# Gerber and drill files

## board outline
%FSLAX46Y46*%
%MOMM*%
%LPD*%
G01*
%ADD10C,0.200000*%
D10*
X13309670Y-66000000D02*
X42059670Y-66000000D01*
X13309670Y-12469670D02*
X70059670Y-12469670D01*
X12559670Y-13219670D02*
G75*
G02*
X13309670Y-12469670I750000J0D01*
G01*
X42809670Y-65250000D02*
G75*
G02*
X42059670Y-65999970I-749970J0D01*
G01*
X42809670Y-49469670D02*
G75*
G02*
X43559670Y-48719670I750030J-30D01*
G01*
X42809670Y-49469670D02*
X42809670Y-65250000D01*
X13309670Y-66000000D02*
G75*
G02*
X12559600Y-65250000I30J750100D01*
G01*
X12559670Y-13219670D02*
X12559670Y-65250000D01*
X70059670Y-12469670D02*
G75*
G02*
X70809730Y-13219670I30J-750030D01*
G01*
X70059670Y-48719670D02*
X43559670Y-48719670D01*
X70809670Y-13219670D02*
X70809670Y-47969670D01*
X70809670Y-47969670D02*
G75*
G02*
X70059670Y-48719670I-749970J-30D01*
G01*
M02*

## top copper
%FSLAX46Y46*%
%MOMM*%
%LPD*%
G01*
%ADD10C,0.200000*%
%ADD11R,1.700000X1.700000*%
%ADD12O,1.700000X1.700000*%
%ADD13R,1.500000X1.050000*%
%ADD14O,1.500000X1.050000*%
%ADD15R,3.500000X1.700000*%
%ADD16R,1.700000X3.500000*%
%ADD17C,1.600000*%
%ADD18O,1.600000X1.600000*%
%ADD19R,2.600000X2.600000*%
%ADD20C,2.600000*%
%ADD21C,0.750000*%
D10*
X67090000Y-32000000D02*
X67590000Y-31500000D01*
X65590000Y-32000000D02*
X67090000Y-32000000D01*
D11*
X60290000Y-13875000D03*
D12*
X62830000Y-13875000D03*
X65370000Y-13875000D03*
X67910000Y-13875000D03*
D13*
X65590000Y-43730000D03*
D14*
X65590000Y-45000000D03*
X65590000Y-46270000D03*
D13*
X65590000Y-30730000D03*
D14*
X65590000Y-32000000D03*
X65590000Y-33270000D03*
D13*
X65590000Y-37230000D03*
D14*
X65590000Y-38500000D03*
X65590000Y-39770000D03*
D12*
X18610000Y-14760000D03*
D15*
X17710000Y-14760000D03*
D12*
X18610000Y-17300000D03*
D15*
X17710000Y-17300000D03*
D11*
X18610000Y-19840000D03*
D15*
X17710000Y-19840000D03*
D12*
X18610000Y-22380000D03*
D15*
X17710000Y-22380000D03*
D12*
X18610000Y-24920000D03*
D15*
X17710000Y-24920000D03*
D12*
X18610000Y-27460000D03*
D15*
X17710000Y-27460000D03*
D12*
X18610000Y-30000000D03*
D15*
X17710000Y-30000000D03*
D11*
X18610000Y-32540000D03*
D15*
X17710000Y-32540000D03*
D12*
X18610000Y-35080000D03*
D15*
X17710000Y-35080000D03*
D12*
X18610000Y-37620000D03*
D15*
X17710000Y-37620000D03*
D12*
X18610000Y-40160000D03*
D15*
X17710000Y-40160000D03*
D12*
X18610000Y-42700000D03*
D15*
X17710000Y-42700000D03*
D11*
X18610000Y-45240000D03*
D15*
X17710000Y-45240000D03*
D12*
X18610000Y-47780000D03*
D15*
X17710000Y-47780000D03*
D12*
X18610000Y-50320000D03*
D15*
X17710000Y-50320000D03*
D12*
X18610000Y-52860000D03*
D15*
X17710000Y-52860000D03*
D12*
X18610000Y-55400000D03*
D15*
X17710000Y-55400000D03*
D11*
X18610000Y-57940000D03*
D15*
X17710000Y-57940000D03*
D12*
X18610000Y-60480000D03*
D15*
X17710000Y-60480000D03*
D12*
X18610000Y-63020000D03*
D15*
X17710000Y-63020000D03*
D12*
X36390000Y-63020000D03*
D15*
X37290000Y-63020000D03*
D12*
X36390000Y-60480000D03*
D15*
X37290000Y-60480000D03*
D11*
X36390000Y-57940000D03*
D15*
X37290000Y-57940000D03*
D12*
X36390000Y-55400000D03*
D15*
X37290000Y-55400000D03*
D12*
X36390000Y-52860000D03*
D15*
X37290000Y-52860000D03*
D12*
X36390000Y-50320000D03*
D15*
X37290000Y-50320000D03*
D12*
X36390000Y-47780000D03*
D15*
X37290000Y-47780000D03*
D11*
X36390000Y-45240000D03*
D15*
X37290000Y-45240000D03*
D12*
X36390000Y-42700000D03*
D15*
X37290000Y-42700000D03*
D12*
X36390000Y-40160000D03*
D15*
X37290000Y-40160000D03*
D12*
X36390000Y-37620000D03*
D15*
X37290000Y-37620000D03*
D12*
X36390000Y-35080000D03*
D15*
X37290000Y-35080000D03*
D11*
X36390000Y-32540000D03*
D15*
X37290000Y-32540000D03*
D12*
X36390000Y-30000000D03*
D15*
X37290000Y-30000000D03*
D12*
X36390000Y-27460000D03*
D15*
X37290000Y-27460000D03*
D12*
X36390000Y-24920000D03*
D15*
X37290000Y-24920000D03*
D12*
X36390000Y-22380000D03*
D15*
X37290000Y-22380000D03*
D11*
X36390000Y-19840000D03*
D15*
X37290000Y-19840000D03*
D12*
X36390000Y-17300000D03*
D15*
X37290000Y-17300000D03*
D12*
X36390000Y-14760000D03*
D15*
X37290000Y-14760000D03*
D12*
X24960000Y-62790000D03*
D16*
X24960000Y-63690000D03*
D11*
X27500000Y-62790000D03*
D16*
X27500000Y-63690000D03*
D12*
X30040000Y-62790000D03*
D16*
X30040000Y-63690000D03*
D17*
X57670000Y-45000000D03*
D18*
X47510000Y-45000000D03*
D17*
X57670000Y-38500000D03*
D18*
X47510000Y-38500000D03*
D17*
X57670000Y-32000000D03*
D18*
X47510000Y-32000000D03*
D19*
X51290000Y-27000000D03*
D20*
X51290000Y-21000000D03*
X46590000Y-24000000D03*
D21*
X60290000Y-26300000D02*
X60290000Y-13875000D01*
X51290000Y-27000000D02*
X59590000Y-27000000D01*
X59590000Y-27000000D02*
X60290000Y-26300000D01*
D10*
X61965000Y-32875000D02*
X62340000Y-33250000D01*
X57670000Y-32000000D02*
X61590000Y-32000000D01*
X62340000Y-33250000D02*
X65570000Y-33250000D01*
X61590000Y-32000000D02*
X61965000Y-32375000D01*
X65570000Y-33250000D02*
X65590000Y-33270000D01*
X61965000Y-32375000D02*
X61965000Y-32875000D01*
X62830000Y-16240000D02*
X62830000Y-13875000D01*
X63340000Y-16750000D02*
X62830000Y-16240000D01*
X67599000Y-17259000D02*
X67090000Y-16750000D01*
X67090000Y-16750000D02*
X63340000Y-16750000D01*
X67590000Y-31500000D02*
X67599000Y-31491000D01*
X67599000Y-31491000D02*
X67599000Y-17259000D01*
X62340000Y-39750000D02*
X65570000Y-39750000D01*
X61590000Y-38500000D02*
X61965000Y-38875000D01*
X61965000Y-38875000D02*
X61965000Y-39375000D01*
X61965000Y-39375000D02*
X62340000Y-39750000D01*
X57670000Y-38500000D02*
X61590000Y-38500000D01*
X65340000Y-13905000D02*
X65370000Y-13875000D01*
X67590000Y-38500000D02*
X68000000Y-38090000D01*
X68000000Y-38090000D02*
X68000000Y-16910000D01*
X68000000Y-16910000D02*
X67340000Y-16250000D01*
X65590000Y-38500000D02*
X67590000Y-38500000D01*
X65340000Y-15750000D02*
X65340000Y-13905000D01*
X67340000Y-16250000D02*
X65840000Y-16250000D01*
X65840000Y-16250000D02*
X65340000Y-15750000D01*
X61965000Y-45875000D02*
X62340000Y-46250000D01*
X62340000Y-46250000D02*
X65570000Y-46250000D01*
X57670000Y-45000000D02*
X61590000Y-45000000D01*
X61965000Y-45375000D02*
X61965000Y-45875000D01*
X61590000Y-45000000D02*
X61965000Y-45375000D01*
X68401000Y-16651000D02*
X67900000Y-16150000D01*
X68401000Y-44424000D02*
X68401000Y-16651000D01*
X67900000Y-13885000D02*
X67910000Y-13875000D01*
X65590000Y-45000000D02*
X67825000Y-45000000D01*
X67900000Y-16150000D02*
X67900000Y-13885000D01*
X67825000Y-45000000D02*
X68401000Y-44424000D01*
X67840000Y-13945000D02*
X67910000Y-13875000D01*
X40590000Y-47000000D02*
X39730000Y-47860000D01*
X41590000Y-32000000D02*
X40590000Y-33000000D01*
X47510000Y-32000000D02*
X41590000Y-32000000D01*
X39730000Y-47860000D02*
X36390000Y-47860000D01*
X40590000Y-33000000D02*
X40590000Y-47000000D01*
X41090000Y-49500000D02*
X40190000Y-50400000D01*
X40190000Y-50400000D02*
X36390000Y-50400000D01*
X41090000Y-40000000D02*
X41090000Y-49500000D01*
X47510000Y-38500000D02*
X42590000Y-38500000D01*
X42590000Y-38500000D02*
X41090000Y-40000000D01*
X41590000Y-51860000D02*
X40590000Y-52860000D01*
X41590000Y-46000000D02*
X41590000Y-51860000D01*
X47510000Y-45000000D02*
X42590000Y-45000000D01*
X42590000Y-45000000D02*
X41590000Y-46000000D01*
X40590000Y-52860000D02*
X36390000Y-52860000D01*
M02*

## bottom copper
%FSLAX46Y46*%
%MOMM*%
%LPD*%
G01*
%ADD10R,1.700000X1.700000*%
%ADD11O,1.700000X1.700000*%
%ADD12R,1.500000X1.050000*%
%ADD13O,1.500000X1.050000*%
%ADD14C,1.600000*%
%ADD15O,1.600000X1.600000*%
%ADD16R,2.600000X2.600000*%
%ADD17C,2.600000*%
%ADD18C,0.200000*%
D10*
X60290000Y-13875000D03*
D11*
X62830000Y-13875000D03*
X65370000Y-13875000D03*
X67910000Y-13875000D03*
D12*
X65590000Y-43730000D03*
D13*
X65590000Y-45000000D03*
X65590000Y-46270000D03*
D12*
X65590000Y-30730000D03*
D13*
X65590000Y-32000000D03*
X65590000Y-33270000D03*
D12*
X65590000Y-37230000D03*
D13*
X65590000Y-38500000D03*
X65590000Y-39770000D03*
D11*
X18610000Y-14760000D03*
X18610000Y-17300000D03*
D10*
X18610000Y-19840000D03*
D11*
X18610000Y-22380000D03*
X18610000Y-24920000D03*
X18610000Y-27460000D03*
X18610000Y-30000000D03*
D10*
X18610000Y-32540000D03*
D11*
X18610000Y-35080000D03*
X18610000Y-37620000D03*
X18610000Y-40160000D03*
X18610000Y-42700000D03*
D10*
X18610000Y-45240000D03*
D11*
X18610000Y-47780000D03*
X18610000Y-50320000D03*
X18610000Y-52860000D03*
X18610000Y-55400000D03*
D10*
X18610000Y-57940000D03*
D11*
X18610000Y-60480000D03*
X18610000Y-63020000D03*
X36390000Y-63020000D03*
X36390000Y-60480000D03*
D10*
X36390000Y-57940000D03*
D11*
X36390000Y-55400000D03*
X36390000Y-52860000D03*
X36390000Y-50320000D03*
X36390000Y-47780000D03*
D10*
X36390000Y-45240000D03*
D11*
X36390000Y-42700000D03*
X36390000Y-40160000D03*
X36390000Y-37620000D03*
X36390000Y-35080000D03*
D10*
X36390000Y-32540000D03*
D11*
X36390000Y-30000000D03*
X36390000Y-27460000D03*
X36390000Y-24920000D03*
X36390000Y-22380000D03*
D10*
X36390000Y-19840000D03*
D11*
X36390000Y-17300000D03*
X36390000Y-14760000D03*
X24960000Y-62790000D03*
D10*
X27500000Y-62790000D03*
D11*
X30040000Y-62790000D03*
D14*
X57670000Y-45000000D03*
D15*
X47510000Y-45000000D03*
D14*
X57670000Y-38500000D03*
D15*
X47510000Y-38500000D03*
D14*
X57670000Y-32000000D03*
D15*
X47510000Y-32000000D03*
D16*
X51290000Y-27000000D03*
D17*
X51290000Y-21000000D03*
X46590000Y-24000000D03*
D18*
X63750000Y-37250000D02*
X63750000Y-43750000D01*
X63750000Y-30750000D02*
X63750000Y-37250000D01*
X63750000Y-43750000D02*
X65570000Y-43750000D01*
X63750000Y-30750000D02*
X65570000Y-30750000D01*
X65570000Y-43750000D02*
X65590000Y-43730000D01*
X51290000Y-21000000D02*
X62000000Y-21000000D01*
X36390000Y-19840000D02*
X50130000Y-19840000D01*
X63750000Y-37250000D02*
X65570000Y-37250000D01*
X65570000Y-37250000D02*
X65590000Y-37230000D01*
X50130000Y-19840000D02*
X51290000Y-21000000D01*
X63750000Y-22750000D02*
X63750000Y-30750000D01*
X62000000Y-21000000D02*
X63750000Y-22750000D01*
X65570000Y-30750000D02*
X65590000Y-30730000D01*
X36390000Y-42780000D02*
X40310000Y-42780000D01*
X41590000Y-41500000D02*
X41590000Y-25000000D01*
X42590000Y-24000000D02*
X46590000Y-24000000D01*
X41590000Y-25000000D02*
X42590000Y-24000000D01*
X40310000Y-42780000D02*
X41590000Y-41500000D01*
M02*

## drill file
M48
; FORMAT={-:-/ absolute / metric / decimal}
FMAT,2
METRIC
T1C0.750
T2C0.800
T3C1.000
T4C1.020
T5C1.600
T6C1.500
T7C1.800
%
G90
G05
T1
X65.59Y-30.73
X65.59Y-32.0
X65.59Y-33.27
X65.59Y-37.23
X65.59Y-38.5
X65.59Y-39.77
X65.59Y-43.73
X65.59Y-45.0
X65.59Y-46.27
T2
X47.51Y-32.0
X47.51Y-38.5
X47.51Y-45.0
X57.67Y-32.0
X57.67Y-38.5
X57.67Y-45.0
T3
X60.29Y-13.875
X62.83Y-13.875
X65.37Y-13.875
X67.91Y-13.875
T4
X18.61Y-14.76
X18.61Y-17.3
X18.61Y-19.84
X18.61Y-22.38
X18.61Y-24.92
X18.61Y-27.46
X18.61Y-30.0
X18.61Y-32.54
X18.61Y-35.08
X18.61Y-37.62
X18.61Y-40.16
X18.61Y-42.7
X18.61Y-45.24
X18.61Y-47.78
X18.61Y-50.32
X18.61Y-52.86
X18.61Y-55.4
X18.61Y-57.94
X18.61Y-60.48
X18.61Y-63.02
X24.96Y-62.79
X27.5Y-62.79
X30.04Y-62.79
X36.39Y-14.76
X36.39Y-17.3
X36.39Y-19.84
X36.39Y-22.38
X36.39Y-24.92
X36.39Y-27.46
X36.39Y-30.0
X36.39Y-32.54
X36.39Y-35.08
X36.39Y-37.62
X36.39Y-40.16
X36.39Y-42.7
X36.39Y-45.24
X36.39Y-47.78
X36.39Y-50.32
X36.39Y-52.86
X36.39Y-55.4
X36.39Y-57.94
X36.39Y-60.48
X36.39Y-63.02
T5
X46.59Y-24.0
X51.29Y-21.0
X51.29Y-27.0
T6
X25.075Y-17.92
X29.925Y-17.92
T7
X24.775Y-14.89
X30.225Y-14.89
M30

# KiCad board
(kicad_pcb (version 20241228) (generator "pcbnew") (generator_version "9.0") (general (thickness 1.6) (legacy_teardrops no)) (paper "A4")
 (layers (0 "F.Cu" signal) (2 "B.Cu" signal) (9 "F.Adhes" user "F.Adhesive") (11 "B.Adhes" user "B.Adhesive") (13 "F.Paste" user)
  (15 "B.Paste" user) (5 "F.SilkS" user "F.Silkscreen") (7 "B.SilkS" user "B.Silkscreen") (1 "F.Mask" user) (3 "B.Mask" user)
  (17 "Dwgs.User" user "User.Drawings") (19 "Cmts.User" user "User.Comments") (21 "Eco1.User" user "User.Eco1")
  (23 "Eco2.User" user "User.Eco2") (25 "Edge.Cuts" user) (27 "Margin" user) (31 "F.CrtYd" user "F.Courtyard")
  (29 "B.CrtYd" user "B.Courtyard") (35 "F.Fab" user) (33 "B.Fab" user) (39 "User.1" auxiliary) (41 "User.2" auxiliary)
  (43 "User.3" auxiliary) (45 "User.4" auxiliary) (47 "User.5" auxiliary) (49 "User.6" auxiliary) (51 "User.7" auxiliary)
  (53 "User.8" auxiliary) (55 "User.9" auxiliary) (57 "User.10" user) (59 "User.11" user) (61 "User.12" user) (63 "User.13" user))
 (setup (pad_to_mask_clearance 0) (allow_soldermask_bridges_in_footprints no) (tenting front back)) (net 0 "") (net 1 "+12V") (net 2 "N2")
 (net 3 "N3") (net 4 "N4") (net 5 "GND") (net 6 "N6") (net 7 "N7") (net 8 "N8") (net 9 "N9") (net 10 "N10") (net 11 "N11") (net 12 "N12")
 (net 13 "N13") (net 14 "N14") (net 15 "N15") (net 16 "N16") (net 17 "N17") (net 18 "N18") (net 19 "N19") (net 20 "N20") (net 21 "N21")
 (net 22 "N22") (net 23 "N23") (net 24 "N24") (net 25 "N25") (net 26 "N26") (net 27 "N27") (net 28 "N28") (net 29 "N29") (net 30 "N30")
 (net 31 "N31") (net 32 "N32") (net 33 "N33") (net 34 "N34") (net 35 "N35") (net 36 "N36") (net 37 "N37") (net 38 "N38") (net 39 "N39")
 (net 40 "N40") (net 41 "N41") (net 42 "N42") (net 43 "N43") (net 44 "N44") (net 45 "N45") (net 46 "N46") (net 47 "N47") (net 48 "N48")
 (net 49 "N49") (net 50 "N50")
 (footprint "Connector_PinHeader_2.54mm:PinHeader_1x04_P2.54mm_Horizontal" (layer "F.Cu") (at 60.29 13.875 90)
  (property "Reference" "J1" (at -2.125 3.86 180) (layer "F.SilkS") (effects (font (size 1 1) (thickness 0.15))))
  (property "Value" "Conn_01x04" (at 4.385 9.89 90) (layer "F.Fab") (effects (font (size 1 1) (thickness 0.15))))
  (pad "1" thru_hole rect (at 0 0 90) (size 1.7 1.7) (drill 1) (layers "*.Cu" "*.Mask") (remove_unused_layers no) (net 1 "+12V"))
  (pad "2" thru_hole oval (at 0 2.54 90) (size 1.7 1.7) (drill 1) (layers "*.Cu" "*.Mask") (remove_unused_layers no) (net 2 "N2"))
  (pad "3" thru_hole oval (at 0 5.08 90) (size 1.7 1.7) (drill 1) (layers "*.Cu" "*.Mask") (remove_unused_layers no) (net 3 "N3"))
  (pad "4" thru_hole oval (at 0 7.62 90) (size 1.7 1.7) (drill 1) (layers "*.Cu" "*.Mask") (remove_unused_layers no) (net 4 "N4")))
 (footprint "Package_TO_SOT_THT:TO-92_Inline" (layer "F.Cu") (at 65.59 43.73 -90)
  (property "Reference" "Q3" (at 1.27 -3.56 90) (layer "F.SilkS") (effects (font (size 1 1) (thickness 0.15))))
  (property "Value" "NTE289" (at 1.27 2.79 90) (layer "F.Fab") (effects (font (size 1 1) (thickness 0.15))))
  (pad "1" thru_hole rect (at 0 0 270) (size 1.05 1.5) (drill 0.75) (layers "*.Cu" "*.Mask") (remove_unused_layers no) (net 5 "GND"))
  (pad "2" thru_hole oval (at 1.27 0 270) (size 1.05 1.5) (drill 0.75) (layers "*.Cu" "*.Mask") (remove_unused_layers no) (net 4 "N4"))
  (pad "3" thru_hole oval (at 2.54 0 270) (size 1.05 1.5) (drill 0.75) (layers "*.Cu" "*.Mask") (remove_unused_layers no) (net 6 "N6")))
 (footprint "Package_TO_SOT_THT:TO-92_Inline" (layer "F.Cu") (at 65.59 30.73 -90)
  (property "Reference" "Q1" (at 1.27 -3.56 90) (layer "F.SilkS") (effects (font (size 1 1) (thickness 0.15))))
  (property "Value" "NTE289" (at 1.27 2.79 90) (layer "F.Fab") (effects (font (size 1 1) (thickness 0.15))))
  (pad "1" thru_hole rect (at 0 0 270) (size 1.05 1.5) (drill 0.75) (layers "*.Cu" "*.Mask") (remove_unused_layers no) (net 5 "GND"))
  (pad "2" thru_hole oval (at 1.27 0 270) (size 1.05 1.5) (drill 0.75) (layers "*.Cu" "*.Mask") (remove_unused_layers no) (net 2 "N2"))
  (pad "3" thru_hole oval (at 2.54 0 270) (size 1.05 1.5) (drill 0.75) (layers "*.Cu" "*.Mask") (remove_unused_layers no) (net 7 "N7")))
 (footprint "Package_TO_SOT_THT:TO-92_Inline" (layer "F.Cu") (at 65.59 37.23 -90)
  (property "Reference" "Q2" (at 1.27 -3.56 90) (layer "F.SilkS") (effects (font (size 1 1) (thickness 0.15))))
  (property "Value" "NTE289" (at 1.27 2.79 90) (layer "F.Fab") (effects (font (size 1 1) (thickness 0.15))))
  (pad "1" thru_hole rect (at 0 0 270) (size 1.05 1.5) (drill 0.75) (layers "*.Cu" "*.Mask") (remove_unused_layers no) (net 5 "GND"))
  (pad "2" thru_hole oval (at 1.27 0 270) (size 1.05 1.5) (drill 0.75) (layers "*.Cu" "*.Mask") (remove_unused_layers no) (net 3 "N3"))
  (pad "3" thru_hole oval (at 2.54 0 270) (size 1.05 1.5) (drill 0.75) (layers "*.Cu" "*.Mask") (remove_unused_layers no) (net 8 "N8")))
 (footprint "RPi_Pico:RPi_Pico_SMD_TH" (layer "F.Cu") (at 27.5 38.89)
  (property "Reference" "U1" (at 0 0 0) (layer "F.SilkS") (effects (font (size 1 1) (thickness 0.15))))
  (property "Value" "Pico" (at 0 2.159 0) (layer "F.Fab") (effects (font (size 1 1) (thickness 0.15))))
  (pad "" np_thru_hole oval (at -2.725 -24) (size 1.8 1.8) (drill 1.8) (layers "*.Cu" "*.Mask"))
  (pad "" np_thru_hole oval (at -2.425 -20.97) (size 1.5 1.5) (drill 1.5) (layers "*.Cu" "*.Mask"))
  (pad "" np_thru_hole oval (at 2.425 -20.97) (size 1.5 1.5) (drill 1.5) (layers "*.Cu" "*.Mask"))
  (pad "" np_thru_hole oval (at 2.725 -24) (size 1.8 1.8) (drill 1.8) (layers "*.Cu" "*.Mask"))
  (pad "1" thru_hole oval (at -8.89 -24.13) (size 1.7 1.7) (drill 1.02) (layers "*.Cu" "*.Mask") (remove_unused_layers no) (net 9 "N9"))
  (pad "1" smd rect (at -8.89 -24.13) (size 3.5 1.7) (drill (offset -0.9 0)) (layers "F.Cu" "F.Mask") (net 9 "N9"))
  (pad "2" thru_hole oval (at -8.89 -21.59) (size 1.7 1.7) (drill 1.02) (layers "*.Cu" "*.Mask") (remove_unused_layers no) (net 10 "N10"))
  (pad "2" smd rect (at -8.89 -21.59) (size 3.5 1.7) (drill (offset -0.9 0)) (layers "F.Cu" "F.Mask") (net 10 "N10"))
  (pad "3" thru_hole rect (at -8.89 -19.05) (size 1.7 1.7) (drill 1.02) (layers "*.Cu" "*.Mask") (remove_unused_layers no) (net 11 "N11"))
  (pad "3" smd rect (at -8.89 -19.05) (size 3.5 1.7) (drill (offset -0.9 0)) (layers "F.Cu" "F.Mask") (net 11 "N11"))
  (pad "4" thru_hole oval (at -8.89 -16.51) (size 1.7 1.7) (drill 1.02) (layers "*.Cu" "*.Mask") (remove_unused_layers no) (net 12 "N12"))
  (pad "4" smd rect (at -8.89 -16.51) (size 3.5 1.7) (drill (offset -0.9 0)) (layers "F.Cu" "F.Mask") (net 12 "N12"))
  (pad "5" thru_hole oval (at -8.89 -13.97) (size 1.7 1.7) (drill 1.02) (layers "*.Cu" "*.Mask") (remove_unused_layers no) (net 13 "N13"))
  (pad "5" smd rect (at -8.89 -13.97) (size 3.5 1.7) (drill (offset -0.9 0)) (layers "F.Cu" "F.Mask") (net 13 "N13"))
  (pad "6" thru_hole oval (at -8.89 -11.43) (size 1.7 1.7) (drill 1.02) (layers "*.Cu" "*.Mask") (remove_unused_layers no) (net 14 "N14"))
  (pad "6" smd rect (at -8.89 -11.43) (size 3.5 1.7) (drill (offset -0.9 0)) (layers "F.Cu" "F.Mask") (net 14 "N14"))
  (pad "7" thru_hole oval (at -8.89 -8.89) (size 1.7 1.7) (drill 1.02) (layers "*.Cu" "*.Mask") (remove_unused_layers no) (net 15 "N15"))
  (pad "7" smd rect (at -8.89 -8.89) (size 3.5 1.7) (drill (offset -0.9 0)) (layers "F.Cu" "F.Mask") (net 15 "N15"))
  (pad "8" thru_hole rect (at -8.89 -6.35) (size 1.7 1.7) (drill 1.02) (layers "*.Cu" "*.Mask") (remove_unused_layers no) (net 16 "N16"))
  (pad "8" smd rect (at -8.89 -6.35) (size 3.5 1.7) (drill (offset -0.9 0)) (layers "F.Cu" "F.Mask") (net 16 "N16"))
  (pad "9" thru_hole oval (at -8.89 -3.81) (size 1.7 1.7) (drill 1.02) (layers "*.Cu" "*.Mask") (remove_unused_layers no) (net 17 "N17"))
  (pad "9" smd rect (at -8.89 -3.81) (size 3.5 1.7) (drill (offset -0.9 0)) (layers "F.Cu" "F.Mask") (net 17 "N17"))
  (pad "10" thru_hole oval (at -8.89 -1.27) (size 1.7 1.7) (drill 1.02) (layers "*.Cu" "*.Mask") (remove_unused_layers no) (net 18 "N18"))
  (pad "10" smd rect (at -8.89 -1.27) (size 3.5 1.7) (drill (offset -0.9 0)) (layers "F.Cu" "F.Mask") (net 18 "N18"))
  (pad "11" thru_hole oval (at -8.89 1.27) (size 1.7 1.7) (drill 1.02) (layers "*.Cu" "*.Mask") (remove_unused_layers no) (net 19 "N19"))
  (pad "11" smd rect (at -8.89 1.27) (size 3.5 1.7) (drill (offset -0.9 0)) (layers "F.Cu" "F.Mask") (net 19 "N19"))
  (pad "12" thru_hole oval (at -8.89 3.81) (size 1.7 1.7) (drill 1.02) (layers "*.Cu" "*.Mask") (remove_unused_layers no) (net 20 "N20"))
  (pad "12" smd rect (at -8.89 3.81) (size 3.5 1.7) (drill (offset -0.9 0)) (layers "F.Cu" "F.Mask") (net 20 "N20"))
  (pad "13" thru_hole rect (at -8.89 6.35) (size 1.7 1.7) (drill 1.02) (layers "*.Cu" "*.Mask") (remove_unused_layers no) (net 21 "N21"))
  (pad "13" smd rect (at -8.89 6.35) (size 3.5 1.7) (drill (offset -0.9 0)) (layers "F.Cu" "F.Mask") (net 21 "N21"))
  (pad "14" thru_hole oval (at -8.89 8.89) (size 1.7 1.7) (drill 1.02) (layers "*.Cu" "*.Mask") (remove_unused_layers no) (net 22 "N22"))
  (pad "14" smd rect (at -8.89 8.89) (size 3.5 1.7) (drill (offset -0.9 0)) (layers "F.Cu" "F.Mask") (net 22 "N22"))
  (pad "15" thru_hole oval (at -8.89 11.43) (size 1.7 1.7) (drill 1.02) (layers "*.Cu" "*.Mask") (remove_unused_layers no) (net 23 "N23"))
  (pad "15" smd rect (at -8.89 11.43) (size 3.5 1.7) (drill (offset -0.9 0)) (layers "F.Cu" "F.Mask") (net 23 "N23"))
  (pad "16" thru_hole oval (at -8.89 13.97) (size 1.7 1.7) (drill 1.02) (layers "*.Cu" "*.Mask") (remove_unused_layers no) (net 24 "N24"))
  (pad "16" smd rect (at -8.89 13.97) (size 3.5 1.7) (drill (offset -0.9 0)) (layers "F.Cu" "F.Mask") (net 24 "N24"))
  (pad "17" thru_hole oval (at -8.89 16.51) (size 1.7 1.7) (drill 1.02) (layers "*.Cu" "*.Mask") (remove_unused_layers no) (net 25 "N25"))
  (pad "17" smd rect (at -8.89 16.51) (size 3.5 1.7) (drill (offset -0.9 0)) (layers "F.Cu" "F.Mask") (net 25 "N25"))
  (pad "18" thru_hole rect (at -8.89 19.05) (size 1.7 1.7) (drill 1.02) (layers "*.Cu" "*.Mask") (remove_unused_layers no) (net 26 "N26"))
  (pad "18" smd rect (at -8.89 19.05) (size 3.5 1.7) (drill (offset -0.9 0)) (layers "F.Cu" "F.Mask") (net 26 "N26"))
  (pad "19" thru_hole oval (at -8.89 21.59) (size 1.7 1.7) (drill 1.02) (layers "*.Cu" "*.Mask") (remove_unused_layers no) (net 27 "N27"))
  (pad "19" smd rect (at -8.89 21.59) (size 3.5 1.7) (drill (offset -0.9 0)) (layers "F.Cu" "F.Mask") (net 27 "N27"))
  (pad "20" thru_hole oval (at -8.89 24.13) (size 1.7 1.7) (drill 1.02) (layers "*.Cu" "*.Mask") (remove_unused_layers no) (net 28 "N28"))
  (pad "20" smd rect (at -8.89 24.13) (size 3.5 1.7) (drill (offset -0.9 0)) (layers "F.Cu" "F.Mask") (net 28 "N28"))
  (pad "21" thru_hole oval (at 8.89 24.13) (size 1.7 1.7) (drill 1.02) (layers "*.Cu" "*.Mask") (remove_unused_layers no) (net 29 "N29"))
  (pad "21" smd rect (at 8.89 24.13) (size 3.5 1.7) (drill (offset 0.9 0)) (layers "F.Cu" "F.Mask") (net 29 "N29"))
  (pad "22" thru_hole oval (at 8.89 21.59) (size 1.7 1.7) (drill 1.02) (layers "*.Cu" "*.Mask") (remove_unused_layers no) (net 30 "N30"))
  (pad "22" smd rect (at 8.89 21.59) (size 3.5 1.7) (drill (offset 0.9 0)) (layers "F.Cu" "F.Mask") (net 30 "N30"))
  (pad "23" thru_hole rect (at 8.89 19.05) (size 1.7 1.7) (drill 1.02) (layers "*.Cu" "*.Mask") (remove_unused_layers no) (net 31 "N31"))
  (pad "23" smd rect (at 8.89 19.05) (size 3.5 1.7) (drill (offset 0.9 0)) (layers "F.Cu" "F.Mask") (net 31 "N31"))
  (pad "24" thru_hole oval (at 8.89 16.51) (size 1.7 1.7) (drill 1.02) (layers "*.Cu" "*.Mask") (remove_unused_layers no) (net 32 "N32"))
  (pad "24" smd rect (at 8.89 16.51) (size 3.5 1.7) (drill (offset 0.9 0)) (layers "F.Cu" "F.Mask") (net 32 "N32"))
  (pad "25" thru_hole oval (at 8.89 13.97) (size 1.7 1.7) (drill 1.02) (layers "*.Cu" "*.Mask") (remove_unused_layers no) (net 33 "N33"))
  (pad "25" smd rect (at 8.89 13.97) (size 3.5 1.7) (drill (offset 0.9 0)) (layers "F.Cu" "F.Mask") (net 33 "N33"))
  (pad "26" thru_hole oval (at 8.89 11.43) (size 1.7 1.7) (drill 1.02) (layers "*.Cu" "*.Mask") (remove_unused_layers no) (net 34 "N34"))
  (pad "26" smd rect (at 8.89 11.43) (size 3.5 1.7) (drill (offset 0.9 0)) (layers "F.Cu" "F.Mask") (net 34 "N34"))
  (pad "27" thru_hole oval (at 8.89 8.89) (size 1.7 1.7) (drill 1.02) (layers "*.Cu" "*.Mask") (remove_unused_layers no) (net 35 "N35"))
  (pad "27" smd rect (at 8.89 8.89) (size 3.5 1.7) (drill (offset 0.9 0)) (layers "F.Cu" "F.Mask") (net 35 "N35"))
  (pad "28" thru_hole rect (at 8.89 6.35) (size 1.7 1.7) (drill 1.02) (layers "*.Cu" "*.Mask") (remove_unused_layers no) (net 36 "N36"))
  (pad "28" smd rect (at 8.89 6.35) (size 3.5 1.7) (drill (offset 0.9 0)) (layers "F.Cu" "F.Mask") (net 36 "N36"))
  (pad "29" thru_hole oval (at 8.89 3.81) (size 1.7 1.7) (drill 1.02) (layers "*.Cu" "*.Mask") (remove_unused_layers no) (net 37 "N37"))
  (pad "29" smd rect (at 8.89 3.81) (size 3.5 1.7) (drill (offset 0.9 0)) (layers "F.Cu" "F.Mask") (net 37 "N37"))
  (pad "30" thru_hole oval (at 8.89 1.27) (size 1.7 1.7) (drill 1.02) (layers "*.Cu" "*.Mask") (remove_unused_layers no) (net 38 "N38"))
  (pad "30" smd rect (at 8.89 1.27) (size 3.5 1.7) (drill (offset 0.9 0)) (layers "F.Cu" "F.Mask") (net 38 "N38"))
  (pad "31" thru_hole oval (at 8.89 -1.27) (size 1.7 1.7) (drill 1.02) (layers "*.Cu" "*.Mask") (remove_unused_layers no) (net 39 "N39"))
  (pad "31" smd rect (at 8.89 -1.27) (size 3.5 1.7) (drill (offset 0.9 0)) (layers "F.Cu" "F.Mask") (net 39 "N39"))
  (pad "32" thru_hole oval (at 8.89 -3.81) (size 1.7 1.7) (drill 1.02) (layers "*.Cu" "*.Mask") (remove_unused_layers no) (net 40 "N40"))
  (pad "32" smd rect (at 8.89 -3.81) (size 3.5 1.7) (drill (offset 0.9 0)) (layers "F.Cu" "F.Mask") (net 40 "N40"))
  (pad "33" thru_hole rect (at 8.89 -6.35) (size 1.7 1.7) (drill 1.02) (layers "*.Cu" "*.Mask") (remove_unused_layers no) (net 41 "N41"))
  (pad "33" smd rect (at 8.89 -6.35) (size 3.5 1.7) (drill (offset 0.9 0)) (layers "F.Cu" "F.Mask") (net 41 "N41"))
  (pad "34" thru_hole oval (at 8.89 -8.89) (size 1.7 1.7) (drill 1.02) (layers "*.Cu" "*.Mask") (remove_unused_layers no) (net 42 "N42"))
  (pad "34" smd rect (at 8.89 -8.89) (size 3.5 1.7) (drill (offset 0.9 0)) (layers "F.Cu" "F.Mask") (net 42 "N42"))
  (pad "35" thru_hole oval (at 8.89 -11.43) (size 1.7 1.7) (drill 1.02) (layers "*.Cu" "*.Mask") (remove_unused_layers no) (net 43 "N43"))
  (pad "35" smd rect (at 8.89 -11.43) (size 3.5 1.7) (drill (offset 0.9 0)) (layers "F.Cu" "F.Mask") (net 43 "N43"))
  (pad "36" thru_hole oval (at 8.89 -13.97) (size 1.7 1.7) (drill 1.02) (layers "*.Cu" "*.Mask") (remove_unused_layers no) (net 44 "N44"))
  (pad "36" smd rect (at 8.89 -13.97) (size 3.5 1.7) (drill (offset 0.9 0)) (layers "F.Cu" "F.Mask") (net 44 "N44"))
  (pad "37" thru_hole oval (at 8.89 -16.51) (size 1.7 1.7) (drill 1.02) (layers "*.Cu" "*.Mask") (remove_unused_layers no) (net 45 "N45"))
  (pad "37" smd rect (at 8.89 -16.51) (size 3.5 1.7) (drill (offset 0.9 0)) (layers "F.Cu" "F.Mask") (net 45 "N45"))
  (pad "38" thru_hole rect (at 8.89 -19.05) (size 1.7 1.7) (drill 1.02) (layers "*.Cu" "*.Mask") (remove_unused_layers no) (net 5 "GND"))
  (pad "38" smd rect (at 8.89 -19.05) (size 3.5 1.7) (drill (offset 0.9 0)) (layers "F.Cu" "F.Mask") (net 5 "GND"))
  (pad "39" thru_hole oval (at 8.89 -21.59) (size 1.7 1.7) (drill 1.02) (layers "*.Cu" "*.Mask") (remove_unused_layers no) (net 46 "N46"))
  (pad "39" smd rect (at 8.89 -21.59) (size 3.5 1.7) (drill (offset 0.9 0)) (layers "F.Cu" "F.Mask") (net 46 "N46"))
  (pad "40" thru_hole oval (at 8.89 -24.13) (size 1.7 1.7) (drill 1.02) (layers "*.Cu" "*.Mask") (remove_unused_layers no) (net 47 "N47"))
  (pad "40" smd rect (at 8.89 -24.13) (size 3.5 1.7) (drill (offset 0.9 0)) (layers "F.Cu" "F.Mask") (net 47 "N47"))
  (pad "41" thru_hole oval (at -2.54 23.9) (size 1.7 1.7) (drill 1.02) (layers "*.Cu" "*.Mask") (remove_unused_layers no) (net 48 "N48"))
  (pad "41" smd rect (at -2.54 23.9 90) (size 3.5 1.7) (drill (offset -0.9 0)) (layers "F.Cu" "F.Mask") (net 48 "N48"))
  (pad "42" thru_hole rect (at 0 23.9) (size 1.7 1.7) (drill 1.02) (layers "*.Cu" "*.Mask") (remove_unused_layers no) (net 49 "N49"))
  (pad "42" smd rect (at 0 23.9 90) (size 3.5 1.7) (drill (offset -0.9 0)) (layers "F.Cu" "F.Mask") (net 49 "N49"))
  (pad "43" thru_hole oval (at 2.54 23.9) (size 1.7 1.7) (drill 1.02) (layers "*.Cu" "*.Mask") (remove_unused_layers no) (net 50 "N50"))
  (pad "43" smd rect (at 2.54 23.9 90) (size 3.5 1.7) (drill (offset -0.9 0)) (layers "F.Cu" "F.Mask") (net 50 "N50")))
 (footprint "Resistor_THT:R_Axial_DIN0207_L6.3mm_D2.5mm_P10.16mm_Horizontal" (layer "F.Cu") (at 57.67 45 180)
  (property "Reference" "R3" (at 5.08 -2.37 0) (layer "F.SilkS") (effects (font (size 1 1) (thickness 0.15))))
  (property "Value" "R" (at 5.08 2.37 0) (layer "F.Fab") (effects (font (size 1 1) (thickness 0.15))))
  (pad "1" thru_hole circle (at 0 0 180) (size 1.6 1.6) (drill 0.8) (layers "*.Cu" "*.Mask") (remove_unused_layers no) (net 6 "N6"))
  (pad "2" thru_hole oval (at 10.16 0 180) (size 1.6 1.6) (drill 0.8) (layers "*.Cu" "*.Mask") (remove_unused_layers no) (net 33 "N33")))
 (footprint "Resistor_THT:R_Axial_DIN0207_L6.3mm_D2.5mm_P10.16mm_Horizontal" (layer "F.Cu") (at 57.67 38.5 180)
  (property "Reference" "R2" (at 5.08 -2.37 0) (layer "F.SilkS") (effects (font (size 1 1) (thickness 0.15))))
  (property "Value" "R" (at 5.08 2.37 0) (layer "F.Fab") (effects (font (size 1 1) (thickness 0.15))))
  (pad "1" thru_hole circle (at 0 0 180) (size 1.6 1.6) (drill 0.8) (layers "*.Cu" "*.Mask") (remove_unused_layers no) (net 8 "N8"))
  (pad "2" thru_hole oval (at 10.16 0 180) (size 1.6 1.6) (drill 0.8) (layers "*.Cu" "*.Mask") (remove_unused_layers no) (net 34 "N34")))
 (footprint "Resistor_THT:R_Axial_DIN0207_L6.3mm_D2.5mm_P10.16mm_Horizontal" (layer "F.Cu") (at 57.67 32 180)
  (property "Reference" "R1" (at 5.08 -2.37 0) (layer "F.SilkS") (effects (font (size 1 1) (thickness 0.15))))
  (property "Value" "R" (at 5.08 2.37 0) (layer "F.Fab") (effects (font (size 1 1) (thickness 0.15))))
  (pad "1" thru_hole circle (at 0 0 180) (size 1.6 1.6) (drill 0.8) (layers "*.Cu" "*.Mask") (remove_unused_layers no) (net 7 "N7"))
  (pad "2" thru_hole oval (at 10.16 0 180) (size 1.6 1.6) (drill 0.8) (layers "*.Cu" "*.Mask") (remove_unused_layers no) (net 35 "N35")))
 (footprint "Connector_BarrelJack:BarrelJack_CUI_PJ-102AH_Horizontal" (layer "F.Cu") (at 51.29 27 180)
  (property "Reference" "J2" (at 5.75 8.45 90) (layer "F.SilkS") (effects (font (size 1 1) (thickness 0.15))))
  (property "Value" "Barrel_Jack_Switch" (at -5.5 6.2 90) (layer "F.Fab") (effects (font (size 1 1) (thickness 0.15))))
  (pad "1" thru_hole rect (at 0 0 180) (size 2.6 2.6) (drill 1.6) (layers "*.Cu" "*.Mask") (remove_unused_layers no) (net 1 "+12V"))
  (pad "2" thru_hole circle (at 0 6 180) (size 2.6 2.6) (drill 1.6) (layers "*.Cu" "*.Mask") (remove_unused_layers no) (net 5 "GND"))
  (pad "3" thru_hole circle (at 4.7 3 180) (size 2.6 2.6) (drill 1.6) (layers "*.Cu" "*.Mask") (remove_unused_layers no) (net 37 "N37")))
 (gr_line (start 67.09 32) (end 67.59 31.5) (stroke (width 0.2) (type default)) (layer "F.Cu") (net 2))
 (gr_line (start 65.59 32) (end 67.09 32) (stroke (width 0.2) (type default)) (layer "F.Cu") (net 2))
 (gr_line (start 13.30967 66) (end 42.05967 66) (stroke (width 0.2) (type default)) (layer "Edge.Cuts"))
 (gr_line (start 13.30967 12.46967) (end 70.05967 12.46967) (stroke (width 0.2) (type default)) (layer "Edge.Cuts"))
 (gr_arc (start 12.55967 13.21967) (mid 12.77934 12.68934) (end 13.30967 12.46967) (stroke (width 0.2) (type default)) (layer "Edge.Cuts"))
 (gr_arc (start 42.80967 65.25) (mid 42.590009 65.780339) (end 42.05967 66) (stroke (width 0.2) (type default)) (layer "Edge.Cuts"))
 (gr_arc (start 42.80967 49.46967) (mid 43.02934 48.93934) (end 43.55967 48.71967) (stroke (width 0.2) (type default)) (layer "Edge.Cuts"))
 (gr_line (start 42.80967 49.46967) (end 42.80967 65.25) (stroke (width 0.2) (type default)) (layer "Edge.Cuts"))
 (gr_arc (start 13.30967 66) (mid 12.77937 65.780318) (end 12.55967 65.25) (stroke (width 0.2) (type default)) (layer "Edge.Cuts"))
 (gr_line (start 12.55967 13.21967) (end 12.55967 65.25) (stroke (width 0.2) (type default)) (layer "Edge.Cuts"))
 (gr_arc (start 70.05967 12.46967) (mid 70.59 12.68934) (end 70.80967 13.21967) (stroke (width 0.2) (type default)) (layer "Edge.Cuts"))
 (gr_line (start 70.05967 48.71967) (end 43.55967 48.71967) (stroke (width 0.2) (type default)) (layer "Edge.Cuts"))
 (gr_line (start 70.80967 13.21967) (end 70.80967 47.96967) (stroke (width 0.2) (type default)) (layer "Edge.Cuts"))
 (gr_arc (start 70.80967 47.96967) (mid 70.59 48.5) (end 70.05967 48.71967) (stroke (width 0.2) (type default)) (layer "Edge.Cuts"))
 (segment (start 60.29 26.3) (end 60.29 13.875) (width 0.75) (layer "F.Cu") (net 1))
 (segment (start 51.29 27) (end 59.59 27) (width 0.75) (layer "F.Cu") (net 1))
 (segment (start 59.59 27) (end 60.29 26.3) (width 0.75) (layer "F.Cu") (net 1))
 (segment (start 63.75 37.25) (end 63.75 43.75) (width 0.2) (layer "B.Cu") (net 5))
 (segment (start 63.75 30.75) (end 63.75 37.25) (width 0.2) (layer "B.Cu") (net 5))
 (segment (start 63.75 43.75) (end 65.57 43.75) (width 0.2) (layer "B.Cu") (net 5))
 (segment (start 63.75 30.75) (end 65.57 30.75) (width 0.2) (layer "B.Cu") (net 5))
 (segment (start 65.57 43.75) (end 65.59 43.73) (width 0.2) (layer "B.Cu") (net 5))
 (segment (start 51.29 21) (end 62 21) (width 0.2) (layer "B.Cu") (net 5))
 (segment (start 36.39 19.84) (end 50.13 19.84) (width 0.2) (layer "B.Cu") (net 5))
 (segment (start 63.75 37.25) (end 65.57 37.25) (width 0.2) (layer "B.Cu") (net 5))
 (segment (start 65.57 37.25) (end 65.59 37.23) (width 0.2) (layer "B.Cu") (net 5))
 (segment (start 50.13 19.84) (end 51.29 21) (width 0.2) (layer "B.Cu") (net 5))
 (segment (start 63.75 22.75) (end 63.75 30.75) (width 0.2) (layer "B.Cu") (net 5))
 (segment (start 62 21) (end 63.75 22.75) (width 0.2) (layer "B.Cu") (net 5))
 (segment (start 65.57 30.75) (end 65.59 30.73) (width 0.2) (layer "B.Cu") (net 5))
 (segment (start 61.965 32.875) (end 62.34 33.25) (width 0.2) (layer "F.Cu") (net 7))
 (segment (start 57.67 32) (end 61.59 32) (width 0.2) (layer "F.Cu") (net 7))
 (segment (start 62.34 33.25) (end 65.57 33.25) (width 0.2) (layer "F.Cu") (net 7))
 (segment (start 61.59 32) (end 61.965 32.375) (width 0.2) (layer "F.Cu") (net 7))
 (segment (start 65.57 33.25) (end 65.59 33.27) (width 0.2) (layer "F.Cu") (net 7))
 (segment (start 61.965 32.375) (end 61.965 32.875) (width 0.2) (layer "F.Cu") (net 7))
 (segment (start 62.83 16.24) (end 62.83 13.875) (width 0.2) (layer "F.Cu") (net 2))
 (segment (start 63.34 16.75) (end 62.83 16.24) (width 0.2) (layer "F.Cu") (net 2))
 (segment (start 67.599 17.259) (end 67.09 16.75) (width 0.2) (layer "F.Cu") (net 2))
 (segment (start 67.09 16.75) (end 63.34 16.75) (width 0.2) (layer "F.Cu") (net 2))
 (segment (start 67.59 31.5) (end 67.599 31.491) (width 0.2) (layer "F.Cu") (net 2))
 (segment (start 67.599 31.491) (end 67.599 17.259) (width 0.2) (layer "F.Cu") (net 2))
 (segment (start 62.34 39.75) (end 65.57 39.75) (width 0.2) (layer "F.Cu") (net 8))
 (segment (start 61.59 38.5) (end 61.965 38.875) (width 0.2) (layer "F.Cu") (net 8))
 (segment (start 61.965 38.875) (end 61.965 39.375) (width 0.2) (layer "F.Cu") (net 8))
 (segment (start 61.965 39.375) (end 62.34 39.75) (width 0.2) (layer "F.Cu") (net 8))
 (segment (start 57.67 38.5) (end 61.59 38.5) (width 0.2) (layer "F.Cu") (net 8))
 (segment (start 65.34 13.905) (end 65.37 13.875) (width 0.2) (layer "F.Cu") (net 3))
 (segment (start 67.59 38.5) (end 68 38.09) (width 0.2) (layer "F.Cu") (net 3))
 (segment (start 68 38.09) (end 68 16.91) (width 0.2) (layer "F.Cu") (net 3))
 (segment (start 68 16.91) (end 67.34 16.25) (width 0.2) (layer "F.Cu") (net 3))
 (segment (start 65.59 38.5) (end 67.59 38.5) (width 0.2) (layer "F.Cu") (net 3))
 (segment (start 65.34 15.75) (end 65.34 13.905) (width 0.2) (layer "F.Cu") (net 3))
 (segment (start 67.34 16.25) (end 65.84 16.25) (width 0.2) (layer "F.Cu") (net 3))
 (segment (start 65.84 16.25) (end 65.34 15.75) (width 0.2) (layer "F.Cu") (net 3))
 (segment (start 61.965 45.875) (end 62.34 46.25) (width 0.2) (layer "F.Cu") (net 6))
 (segment (start 62.34 46.25) (end 65.57 46.25) (width 0.2) (layer "F.Cu") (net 6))
 (segment (start 57.67 45) (end 61.59 45) (width 0.2) (layer "F.Cu") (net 6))
 (segment (start 61.965 45.375) (end 61.965 45.875) (width 0.2) (layer "F.Cu") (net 6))
 (segment (start 61.59 45) (end 61.965 45.375) (width 0.2) (layer "F.Cu") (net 6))
 (segment (start 68.401 16.651) (end 67.9 16.15) (width 0.2) (layer "F.Cu") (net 4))
 (segment (start 68.401 44.424) (end 68.401 16.651) (width 0.2) (layer "F.Cu") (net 4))
 (segment (start 67.9 13.885) (end 67.91 13.875) (width 0.2) (layer "F.Cu") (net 4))
 (segment (start 65.59 45) (end 67.825 45) (width 0.2) (layer "F.Cu") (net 4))
 (segment (start 67.9 16.15) (end 67.9 13.885) (width 0.2) (layer "F.Cu") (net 4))
 (segment (start 67.825 45) (end 68.401 44.424) (width 0.2) (layer "F.Cu") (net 4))
 (segment (start 67.84 13.945) (end 67.91 13.875) (width 0.2) (layer "F.Cu") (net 4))
 (segment (start 36.39 42.78) (end 40.31 42.78) (width 0.2) (layer "B.Cu") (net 37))
 (segment (start 41.59 41.5) (end 41.59 25) (width 0.2) (layer "B.Cu") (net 37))
 (segment (start 42.59 24) (end 46.59 24) (width 0.2) (layer "B.Cu") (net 37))
 (segment (start 41.59 25) (end 42.59 24) (width 0.2) (layer "B.Cu") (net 37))
 (segment (start 40.31 42.78) (end 41.59 41.5) (width 0.2) (layer "B.Cu") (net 37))
 (segment (start 40.59 47) (end 39.73 47.86) (width 0.2) (layer "F.Cu") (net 35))
 (segment (start 41.59 32) (end 40.59 33) (width 0.2) (layer "F.Cu") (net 35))
 (segment (start 47.51 32) (end 41.59 32) (width 0.2) (layer "F.Cu") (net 35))
 (segment (start 39.73 47.86) (end 36.39 47.86) (width 0.2) (layer "F.Cu") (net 35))
 (segment (start 40.59 33) (end 40.59 47) (width 0.2) (layer "F.Cu") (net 35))
 (segment (start 41.09 49.5) (end 40.19 50.4) (width 0.2) (layer "F.Cu") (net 34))
 (segment (start 40.19 50.4) (end 36.39 50.4) (width 0.2) (layer "F.Cu") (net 34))
 (segment (start 41.09 40) (end 41.09 49.5) (width 0.2) (layer "F.Cu") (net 34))
 (segment (start 47.51 38.5) (end 42.59 38.5) (width 0.2) (layer "F.Cu") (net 34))
 (segment (start 42.59 38.5) (end 41.09 40) (width 0.2) (layer "F.Cu") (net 34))
 (segment (start 41.59 51.86) (end 40.59 52.86) (width 0.2) (layer "F.Cu") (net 33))
 (segment (start 41.59 46) (end 41.59 51.86) (width 0.2) (layer "F.Cu") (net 33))
 (segment (start 47.51 45) (end 42.59 45) (width 0.2) (layer "F.Cu") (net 33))
 (segment (start 42.59 45) (end 41.59 46) (width 0.2) (layer "F.Cu") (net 33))
 (segment (start 40.59 52.86) (end 36.39 52.86) (width 0.2) (layer "F.Cu") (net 33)))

